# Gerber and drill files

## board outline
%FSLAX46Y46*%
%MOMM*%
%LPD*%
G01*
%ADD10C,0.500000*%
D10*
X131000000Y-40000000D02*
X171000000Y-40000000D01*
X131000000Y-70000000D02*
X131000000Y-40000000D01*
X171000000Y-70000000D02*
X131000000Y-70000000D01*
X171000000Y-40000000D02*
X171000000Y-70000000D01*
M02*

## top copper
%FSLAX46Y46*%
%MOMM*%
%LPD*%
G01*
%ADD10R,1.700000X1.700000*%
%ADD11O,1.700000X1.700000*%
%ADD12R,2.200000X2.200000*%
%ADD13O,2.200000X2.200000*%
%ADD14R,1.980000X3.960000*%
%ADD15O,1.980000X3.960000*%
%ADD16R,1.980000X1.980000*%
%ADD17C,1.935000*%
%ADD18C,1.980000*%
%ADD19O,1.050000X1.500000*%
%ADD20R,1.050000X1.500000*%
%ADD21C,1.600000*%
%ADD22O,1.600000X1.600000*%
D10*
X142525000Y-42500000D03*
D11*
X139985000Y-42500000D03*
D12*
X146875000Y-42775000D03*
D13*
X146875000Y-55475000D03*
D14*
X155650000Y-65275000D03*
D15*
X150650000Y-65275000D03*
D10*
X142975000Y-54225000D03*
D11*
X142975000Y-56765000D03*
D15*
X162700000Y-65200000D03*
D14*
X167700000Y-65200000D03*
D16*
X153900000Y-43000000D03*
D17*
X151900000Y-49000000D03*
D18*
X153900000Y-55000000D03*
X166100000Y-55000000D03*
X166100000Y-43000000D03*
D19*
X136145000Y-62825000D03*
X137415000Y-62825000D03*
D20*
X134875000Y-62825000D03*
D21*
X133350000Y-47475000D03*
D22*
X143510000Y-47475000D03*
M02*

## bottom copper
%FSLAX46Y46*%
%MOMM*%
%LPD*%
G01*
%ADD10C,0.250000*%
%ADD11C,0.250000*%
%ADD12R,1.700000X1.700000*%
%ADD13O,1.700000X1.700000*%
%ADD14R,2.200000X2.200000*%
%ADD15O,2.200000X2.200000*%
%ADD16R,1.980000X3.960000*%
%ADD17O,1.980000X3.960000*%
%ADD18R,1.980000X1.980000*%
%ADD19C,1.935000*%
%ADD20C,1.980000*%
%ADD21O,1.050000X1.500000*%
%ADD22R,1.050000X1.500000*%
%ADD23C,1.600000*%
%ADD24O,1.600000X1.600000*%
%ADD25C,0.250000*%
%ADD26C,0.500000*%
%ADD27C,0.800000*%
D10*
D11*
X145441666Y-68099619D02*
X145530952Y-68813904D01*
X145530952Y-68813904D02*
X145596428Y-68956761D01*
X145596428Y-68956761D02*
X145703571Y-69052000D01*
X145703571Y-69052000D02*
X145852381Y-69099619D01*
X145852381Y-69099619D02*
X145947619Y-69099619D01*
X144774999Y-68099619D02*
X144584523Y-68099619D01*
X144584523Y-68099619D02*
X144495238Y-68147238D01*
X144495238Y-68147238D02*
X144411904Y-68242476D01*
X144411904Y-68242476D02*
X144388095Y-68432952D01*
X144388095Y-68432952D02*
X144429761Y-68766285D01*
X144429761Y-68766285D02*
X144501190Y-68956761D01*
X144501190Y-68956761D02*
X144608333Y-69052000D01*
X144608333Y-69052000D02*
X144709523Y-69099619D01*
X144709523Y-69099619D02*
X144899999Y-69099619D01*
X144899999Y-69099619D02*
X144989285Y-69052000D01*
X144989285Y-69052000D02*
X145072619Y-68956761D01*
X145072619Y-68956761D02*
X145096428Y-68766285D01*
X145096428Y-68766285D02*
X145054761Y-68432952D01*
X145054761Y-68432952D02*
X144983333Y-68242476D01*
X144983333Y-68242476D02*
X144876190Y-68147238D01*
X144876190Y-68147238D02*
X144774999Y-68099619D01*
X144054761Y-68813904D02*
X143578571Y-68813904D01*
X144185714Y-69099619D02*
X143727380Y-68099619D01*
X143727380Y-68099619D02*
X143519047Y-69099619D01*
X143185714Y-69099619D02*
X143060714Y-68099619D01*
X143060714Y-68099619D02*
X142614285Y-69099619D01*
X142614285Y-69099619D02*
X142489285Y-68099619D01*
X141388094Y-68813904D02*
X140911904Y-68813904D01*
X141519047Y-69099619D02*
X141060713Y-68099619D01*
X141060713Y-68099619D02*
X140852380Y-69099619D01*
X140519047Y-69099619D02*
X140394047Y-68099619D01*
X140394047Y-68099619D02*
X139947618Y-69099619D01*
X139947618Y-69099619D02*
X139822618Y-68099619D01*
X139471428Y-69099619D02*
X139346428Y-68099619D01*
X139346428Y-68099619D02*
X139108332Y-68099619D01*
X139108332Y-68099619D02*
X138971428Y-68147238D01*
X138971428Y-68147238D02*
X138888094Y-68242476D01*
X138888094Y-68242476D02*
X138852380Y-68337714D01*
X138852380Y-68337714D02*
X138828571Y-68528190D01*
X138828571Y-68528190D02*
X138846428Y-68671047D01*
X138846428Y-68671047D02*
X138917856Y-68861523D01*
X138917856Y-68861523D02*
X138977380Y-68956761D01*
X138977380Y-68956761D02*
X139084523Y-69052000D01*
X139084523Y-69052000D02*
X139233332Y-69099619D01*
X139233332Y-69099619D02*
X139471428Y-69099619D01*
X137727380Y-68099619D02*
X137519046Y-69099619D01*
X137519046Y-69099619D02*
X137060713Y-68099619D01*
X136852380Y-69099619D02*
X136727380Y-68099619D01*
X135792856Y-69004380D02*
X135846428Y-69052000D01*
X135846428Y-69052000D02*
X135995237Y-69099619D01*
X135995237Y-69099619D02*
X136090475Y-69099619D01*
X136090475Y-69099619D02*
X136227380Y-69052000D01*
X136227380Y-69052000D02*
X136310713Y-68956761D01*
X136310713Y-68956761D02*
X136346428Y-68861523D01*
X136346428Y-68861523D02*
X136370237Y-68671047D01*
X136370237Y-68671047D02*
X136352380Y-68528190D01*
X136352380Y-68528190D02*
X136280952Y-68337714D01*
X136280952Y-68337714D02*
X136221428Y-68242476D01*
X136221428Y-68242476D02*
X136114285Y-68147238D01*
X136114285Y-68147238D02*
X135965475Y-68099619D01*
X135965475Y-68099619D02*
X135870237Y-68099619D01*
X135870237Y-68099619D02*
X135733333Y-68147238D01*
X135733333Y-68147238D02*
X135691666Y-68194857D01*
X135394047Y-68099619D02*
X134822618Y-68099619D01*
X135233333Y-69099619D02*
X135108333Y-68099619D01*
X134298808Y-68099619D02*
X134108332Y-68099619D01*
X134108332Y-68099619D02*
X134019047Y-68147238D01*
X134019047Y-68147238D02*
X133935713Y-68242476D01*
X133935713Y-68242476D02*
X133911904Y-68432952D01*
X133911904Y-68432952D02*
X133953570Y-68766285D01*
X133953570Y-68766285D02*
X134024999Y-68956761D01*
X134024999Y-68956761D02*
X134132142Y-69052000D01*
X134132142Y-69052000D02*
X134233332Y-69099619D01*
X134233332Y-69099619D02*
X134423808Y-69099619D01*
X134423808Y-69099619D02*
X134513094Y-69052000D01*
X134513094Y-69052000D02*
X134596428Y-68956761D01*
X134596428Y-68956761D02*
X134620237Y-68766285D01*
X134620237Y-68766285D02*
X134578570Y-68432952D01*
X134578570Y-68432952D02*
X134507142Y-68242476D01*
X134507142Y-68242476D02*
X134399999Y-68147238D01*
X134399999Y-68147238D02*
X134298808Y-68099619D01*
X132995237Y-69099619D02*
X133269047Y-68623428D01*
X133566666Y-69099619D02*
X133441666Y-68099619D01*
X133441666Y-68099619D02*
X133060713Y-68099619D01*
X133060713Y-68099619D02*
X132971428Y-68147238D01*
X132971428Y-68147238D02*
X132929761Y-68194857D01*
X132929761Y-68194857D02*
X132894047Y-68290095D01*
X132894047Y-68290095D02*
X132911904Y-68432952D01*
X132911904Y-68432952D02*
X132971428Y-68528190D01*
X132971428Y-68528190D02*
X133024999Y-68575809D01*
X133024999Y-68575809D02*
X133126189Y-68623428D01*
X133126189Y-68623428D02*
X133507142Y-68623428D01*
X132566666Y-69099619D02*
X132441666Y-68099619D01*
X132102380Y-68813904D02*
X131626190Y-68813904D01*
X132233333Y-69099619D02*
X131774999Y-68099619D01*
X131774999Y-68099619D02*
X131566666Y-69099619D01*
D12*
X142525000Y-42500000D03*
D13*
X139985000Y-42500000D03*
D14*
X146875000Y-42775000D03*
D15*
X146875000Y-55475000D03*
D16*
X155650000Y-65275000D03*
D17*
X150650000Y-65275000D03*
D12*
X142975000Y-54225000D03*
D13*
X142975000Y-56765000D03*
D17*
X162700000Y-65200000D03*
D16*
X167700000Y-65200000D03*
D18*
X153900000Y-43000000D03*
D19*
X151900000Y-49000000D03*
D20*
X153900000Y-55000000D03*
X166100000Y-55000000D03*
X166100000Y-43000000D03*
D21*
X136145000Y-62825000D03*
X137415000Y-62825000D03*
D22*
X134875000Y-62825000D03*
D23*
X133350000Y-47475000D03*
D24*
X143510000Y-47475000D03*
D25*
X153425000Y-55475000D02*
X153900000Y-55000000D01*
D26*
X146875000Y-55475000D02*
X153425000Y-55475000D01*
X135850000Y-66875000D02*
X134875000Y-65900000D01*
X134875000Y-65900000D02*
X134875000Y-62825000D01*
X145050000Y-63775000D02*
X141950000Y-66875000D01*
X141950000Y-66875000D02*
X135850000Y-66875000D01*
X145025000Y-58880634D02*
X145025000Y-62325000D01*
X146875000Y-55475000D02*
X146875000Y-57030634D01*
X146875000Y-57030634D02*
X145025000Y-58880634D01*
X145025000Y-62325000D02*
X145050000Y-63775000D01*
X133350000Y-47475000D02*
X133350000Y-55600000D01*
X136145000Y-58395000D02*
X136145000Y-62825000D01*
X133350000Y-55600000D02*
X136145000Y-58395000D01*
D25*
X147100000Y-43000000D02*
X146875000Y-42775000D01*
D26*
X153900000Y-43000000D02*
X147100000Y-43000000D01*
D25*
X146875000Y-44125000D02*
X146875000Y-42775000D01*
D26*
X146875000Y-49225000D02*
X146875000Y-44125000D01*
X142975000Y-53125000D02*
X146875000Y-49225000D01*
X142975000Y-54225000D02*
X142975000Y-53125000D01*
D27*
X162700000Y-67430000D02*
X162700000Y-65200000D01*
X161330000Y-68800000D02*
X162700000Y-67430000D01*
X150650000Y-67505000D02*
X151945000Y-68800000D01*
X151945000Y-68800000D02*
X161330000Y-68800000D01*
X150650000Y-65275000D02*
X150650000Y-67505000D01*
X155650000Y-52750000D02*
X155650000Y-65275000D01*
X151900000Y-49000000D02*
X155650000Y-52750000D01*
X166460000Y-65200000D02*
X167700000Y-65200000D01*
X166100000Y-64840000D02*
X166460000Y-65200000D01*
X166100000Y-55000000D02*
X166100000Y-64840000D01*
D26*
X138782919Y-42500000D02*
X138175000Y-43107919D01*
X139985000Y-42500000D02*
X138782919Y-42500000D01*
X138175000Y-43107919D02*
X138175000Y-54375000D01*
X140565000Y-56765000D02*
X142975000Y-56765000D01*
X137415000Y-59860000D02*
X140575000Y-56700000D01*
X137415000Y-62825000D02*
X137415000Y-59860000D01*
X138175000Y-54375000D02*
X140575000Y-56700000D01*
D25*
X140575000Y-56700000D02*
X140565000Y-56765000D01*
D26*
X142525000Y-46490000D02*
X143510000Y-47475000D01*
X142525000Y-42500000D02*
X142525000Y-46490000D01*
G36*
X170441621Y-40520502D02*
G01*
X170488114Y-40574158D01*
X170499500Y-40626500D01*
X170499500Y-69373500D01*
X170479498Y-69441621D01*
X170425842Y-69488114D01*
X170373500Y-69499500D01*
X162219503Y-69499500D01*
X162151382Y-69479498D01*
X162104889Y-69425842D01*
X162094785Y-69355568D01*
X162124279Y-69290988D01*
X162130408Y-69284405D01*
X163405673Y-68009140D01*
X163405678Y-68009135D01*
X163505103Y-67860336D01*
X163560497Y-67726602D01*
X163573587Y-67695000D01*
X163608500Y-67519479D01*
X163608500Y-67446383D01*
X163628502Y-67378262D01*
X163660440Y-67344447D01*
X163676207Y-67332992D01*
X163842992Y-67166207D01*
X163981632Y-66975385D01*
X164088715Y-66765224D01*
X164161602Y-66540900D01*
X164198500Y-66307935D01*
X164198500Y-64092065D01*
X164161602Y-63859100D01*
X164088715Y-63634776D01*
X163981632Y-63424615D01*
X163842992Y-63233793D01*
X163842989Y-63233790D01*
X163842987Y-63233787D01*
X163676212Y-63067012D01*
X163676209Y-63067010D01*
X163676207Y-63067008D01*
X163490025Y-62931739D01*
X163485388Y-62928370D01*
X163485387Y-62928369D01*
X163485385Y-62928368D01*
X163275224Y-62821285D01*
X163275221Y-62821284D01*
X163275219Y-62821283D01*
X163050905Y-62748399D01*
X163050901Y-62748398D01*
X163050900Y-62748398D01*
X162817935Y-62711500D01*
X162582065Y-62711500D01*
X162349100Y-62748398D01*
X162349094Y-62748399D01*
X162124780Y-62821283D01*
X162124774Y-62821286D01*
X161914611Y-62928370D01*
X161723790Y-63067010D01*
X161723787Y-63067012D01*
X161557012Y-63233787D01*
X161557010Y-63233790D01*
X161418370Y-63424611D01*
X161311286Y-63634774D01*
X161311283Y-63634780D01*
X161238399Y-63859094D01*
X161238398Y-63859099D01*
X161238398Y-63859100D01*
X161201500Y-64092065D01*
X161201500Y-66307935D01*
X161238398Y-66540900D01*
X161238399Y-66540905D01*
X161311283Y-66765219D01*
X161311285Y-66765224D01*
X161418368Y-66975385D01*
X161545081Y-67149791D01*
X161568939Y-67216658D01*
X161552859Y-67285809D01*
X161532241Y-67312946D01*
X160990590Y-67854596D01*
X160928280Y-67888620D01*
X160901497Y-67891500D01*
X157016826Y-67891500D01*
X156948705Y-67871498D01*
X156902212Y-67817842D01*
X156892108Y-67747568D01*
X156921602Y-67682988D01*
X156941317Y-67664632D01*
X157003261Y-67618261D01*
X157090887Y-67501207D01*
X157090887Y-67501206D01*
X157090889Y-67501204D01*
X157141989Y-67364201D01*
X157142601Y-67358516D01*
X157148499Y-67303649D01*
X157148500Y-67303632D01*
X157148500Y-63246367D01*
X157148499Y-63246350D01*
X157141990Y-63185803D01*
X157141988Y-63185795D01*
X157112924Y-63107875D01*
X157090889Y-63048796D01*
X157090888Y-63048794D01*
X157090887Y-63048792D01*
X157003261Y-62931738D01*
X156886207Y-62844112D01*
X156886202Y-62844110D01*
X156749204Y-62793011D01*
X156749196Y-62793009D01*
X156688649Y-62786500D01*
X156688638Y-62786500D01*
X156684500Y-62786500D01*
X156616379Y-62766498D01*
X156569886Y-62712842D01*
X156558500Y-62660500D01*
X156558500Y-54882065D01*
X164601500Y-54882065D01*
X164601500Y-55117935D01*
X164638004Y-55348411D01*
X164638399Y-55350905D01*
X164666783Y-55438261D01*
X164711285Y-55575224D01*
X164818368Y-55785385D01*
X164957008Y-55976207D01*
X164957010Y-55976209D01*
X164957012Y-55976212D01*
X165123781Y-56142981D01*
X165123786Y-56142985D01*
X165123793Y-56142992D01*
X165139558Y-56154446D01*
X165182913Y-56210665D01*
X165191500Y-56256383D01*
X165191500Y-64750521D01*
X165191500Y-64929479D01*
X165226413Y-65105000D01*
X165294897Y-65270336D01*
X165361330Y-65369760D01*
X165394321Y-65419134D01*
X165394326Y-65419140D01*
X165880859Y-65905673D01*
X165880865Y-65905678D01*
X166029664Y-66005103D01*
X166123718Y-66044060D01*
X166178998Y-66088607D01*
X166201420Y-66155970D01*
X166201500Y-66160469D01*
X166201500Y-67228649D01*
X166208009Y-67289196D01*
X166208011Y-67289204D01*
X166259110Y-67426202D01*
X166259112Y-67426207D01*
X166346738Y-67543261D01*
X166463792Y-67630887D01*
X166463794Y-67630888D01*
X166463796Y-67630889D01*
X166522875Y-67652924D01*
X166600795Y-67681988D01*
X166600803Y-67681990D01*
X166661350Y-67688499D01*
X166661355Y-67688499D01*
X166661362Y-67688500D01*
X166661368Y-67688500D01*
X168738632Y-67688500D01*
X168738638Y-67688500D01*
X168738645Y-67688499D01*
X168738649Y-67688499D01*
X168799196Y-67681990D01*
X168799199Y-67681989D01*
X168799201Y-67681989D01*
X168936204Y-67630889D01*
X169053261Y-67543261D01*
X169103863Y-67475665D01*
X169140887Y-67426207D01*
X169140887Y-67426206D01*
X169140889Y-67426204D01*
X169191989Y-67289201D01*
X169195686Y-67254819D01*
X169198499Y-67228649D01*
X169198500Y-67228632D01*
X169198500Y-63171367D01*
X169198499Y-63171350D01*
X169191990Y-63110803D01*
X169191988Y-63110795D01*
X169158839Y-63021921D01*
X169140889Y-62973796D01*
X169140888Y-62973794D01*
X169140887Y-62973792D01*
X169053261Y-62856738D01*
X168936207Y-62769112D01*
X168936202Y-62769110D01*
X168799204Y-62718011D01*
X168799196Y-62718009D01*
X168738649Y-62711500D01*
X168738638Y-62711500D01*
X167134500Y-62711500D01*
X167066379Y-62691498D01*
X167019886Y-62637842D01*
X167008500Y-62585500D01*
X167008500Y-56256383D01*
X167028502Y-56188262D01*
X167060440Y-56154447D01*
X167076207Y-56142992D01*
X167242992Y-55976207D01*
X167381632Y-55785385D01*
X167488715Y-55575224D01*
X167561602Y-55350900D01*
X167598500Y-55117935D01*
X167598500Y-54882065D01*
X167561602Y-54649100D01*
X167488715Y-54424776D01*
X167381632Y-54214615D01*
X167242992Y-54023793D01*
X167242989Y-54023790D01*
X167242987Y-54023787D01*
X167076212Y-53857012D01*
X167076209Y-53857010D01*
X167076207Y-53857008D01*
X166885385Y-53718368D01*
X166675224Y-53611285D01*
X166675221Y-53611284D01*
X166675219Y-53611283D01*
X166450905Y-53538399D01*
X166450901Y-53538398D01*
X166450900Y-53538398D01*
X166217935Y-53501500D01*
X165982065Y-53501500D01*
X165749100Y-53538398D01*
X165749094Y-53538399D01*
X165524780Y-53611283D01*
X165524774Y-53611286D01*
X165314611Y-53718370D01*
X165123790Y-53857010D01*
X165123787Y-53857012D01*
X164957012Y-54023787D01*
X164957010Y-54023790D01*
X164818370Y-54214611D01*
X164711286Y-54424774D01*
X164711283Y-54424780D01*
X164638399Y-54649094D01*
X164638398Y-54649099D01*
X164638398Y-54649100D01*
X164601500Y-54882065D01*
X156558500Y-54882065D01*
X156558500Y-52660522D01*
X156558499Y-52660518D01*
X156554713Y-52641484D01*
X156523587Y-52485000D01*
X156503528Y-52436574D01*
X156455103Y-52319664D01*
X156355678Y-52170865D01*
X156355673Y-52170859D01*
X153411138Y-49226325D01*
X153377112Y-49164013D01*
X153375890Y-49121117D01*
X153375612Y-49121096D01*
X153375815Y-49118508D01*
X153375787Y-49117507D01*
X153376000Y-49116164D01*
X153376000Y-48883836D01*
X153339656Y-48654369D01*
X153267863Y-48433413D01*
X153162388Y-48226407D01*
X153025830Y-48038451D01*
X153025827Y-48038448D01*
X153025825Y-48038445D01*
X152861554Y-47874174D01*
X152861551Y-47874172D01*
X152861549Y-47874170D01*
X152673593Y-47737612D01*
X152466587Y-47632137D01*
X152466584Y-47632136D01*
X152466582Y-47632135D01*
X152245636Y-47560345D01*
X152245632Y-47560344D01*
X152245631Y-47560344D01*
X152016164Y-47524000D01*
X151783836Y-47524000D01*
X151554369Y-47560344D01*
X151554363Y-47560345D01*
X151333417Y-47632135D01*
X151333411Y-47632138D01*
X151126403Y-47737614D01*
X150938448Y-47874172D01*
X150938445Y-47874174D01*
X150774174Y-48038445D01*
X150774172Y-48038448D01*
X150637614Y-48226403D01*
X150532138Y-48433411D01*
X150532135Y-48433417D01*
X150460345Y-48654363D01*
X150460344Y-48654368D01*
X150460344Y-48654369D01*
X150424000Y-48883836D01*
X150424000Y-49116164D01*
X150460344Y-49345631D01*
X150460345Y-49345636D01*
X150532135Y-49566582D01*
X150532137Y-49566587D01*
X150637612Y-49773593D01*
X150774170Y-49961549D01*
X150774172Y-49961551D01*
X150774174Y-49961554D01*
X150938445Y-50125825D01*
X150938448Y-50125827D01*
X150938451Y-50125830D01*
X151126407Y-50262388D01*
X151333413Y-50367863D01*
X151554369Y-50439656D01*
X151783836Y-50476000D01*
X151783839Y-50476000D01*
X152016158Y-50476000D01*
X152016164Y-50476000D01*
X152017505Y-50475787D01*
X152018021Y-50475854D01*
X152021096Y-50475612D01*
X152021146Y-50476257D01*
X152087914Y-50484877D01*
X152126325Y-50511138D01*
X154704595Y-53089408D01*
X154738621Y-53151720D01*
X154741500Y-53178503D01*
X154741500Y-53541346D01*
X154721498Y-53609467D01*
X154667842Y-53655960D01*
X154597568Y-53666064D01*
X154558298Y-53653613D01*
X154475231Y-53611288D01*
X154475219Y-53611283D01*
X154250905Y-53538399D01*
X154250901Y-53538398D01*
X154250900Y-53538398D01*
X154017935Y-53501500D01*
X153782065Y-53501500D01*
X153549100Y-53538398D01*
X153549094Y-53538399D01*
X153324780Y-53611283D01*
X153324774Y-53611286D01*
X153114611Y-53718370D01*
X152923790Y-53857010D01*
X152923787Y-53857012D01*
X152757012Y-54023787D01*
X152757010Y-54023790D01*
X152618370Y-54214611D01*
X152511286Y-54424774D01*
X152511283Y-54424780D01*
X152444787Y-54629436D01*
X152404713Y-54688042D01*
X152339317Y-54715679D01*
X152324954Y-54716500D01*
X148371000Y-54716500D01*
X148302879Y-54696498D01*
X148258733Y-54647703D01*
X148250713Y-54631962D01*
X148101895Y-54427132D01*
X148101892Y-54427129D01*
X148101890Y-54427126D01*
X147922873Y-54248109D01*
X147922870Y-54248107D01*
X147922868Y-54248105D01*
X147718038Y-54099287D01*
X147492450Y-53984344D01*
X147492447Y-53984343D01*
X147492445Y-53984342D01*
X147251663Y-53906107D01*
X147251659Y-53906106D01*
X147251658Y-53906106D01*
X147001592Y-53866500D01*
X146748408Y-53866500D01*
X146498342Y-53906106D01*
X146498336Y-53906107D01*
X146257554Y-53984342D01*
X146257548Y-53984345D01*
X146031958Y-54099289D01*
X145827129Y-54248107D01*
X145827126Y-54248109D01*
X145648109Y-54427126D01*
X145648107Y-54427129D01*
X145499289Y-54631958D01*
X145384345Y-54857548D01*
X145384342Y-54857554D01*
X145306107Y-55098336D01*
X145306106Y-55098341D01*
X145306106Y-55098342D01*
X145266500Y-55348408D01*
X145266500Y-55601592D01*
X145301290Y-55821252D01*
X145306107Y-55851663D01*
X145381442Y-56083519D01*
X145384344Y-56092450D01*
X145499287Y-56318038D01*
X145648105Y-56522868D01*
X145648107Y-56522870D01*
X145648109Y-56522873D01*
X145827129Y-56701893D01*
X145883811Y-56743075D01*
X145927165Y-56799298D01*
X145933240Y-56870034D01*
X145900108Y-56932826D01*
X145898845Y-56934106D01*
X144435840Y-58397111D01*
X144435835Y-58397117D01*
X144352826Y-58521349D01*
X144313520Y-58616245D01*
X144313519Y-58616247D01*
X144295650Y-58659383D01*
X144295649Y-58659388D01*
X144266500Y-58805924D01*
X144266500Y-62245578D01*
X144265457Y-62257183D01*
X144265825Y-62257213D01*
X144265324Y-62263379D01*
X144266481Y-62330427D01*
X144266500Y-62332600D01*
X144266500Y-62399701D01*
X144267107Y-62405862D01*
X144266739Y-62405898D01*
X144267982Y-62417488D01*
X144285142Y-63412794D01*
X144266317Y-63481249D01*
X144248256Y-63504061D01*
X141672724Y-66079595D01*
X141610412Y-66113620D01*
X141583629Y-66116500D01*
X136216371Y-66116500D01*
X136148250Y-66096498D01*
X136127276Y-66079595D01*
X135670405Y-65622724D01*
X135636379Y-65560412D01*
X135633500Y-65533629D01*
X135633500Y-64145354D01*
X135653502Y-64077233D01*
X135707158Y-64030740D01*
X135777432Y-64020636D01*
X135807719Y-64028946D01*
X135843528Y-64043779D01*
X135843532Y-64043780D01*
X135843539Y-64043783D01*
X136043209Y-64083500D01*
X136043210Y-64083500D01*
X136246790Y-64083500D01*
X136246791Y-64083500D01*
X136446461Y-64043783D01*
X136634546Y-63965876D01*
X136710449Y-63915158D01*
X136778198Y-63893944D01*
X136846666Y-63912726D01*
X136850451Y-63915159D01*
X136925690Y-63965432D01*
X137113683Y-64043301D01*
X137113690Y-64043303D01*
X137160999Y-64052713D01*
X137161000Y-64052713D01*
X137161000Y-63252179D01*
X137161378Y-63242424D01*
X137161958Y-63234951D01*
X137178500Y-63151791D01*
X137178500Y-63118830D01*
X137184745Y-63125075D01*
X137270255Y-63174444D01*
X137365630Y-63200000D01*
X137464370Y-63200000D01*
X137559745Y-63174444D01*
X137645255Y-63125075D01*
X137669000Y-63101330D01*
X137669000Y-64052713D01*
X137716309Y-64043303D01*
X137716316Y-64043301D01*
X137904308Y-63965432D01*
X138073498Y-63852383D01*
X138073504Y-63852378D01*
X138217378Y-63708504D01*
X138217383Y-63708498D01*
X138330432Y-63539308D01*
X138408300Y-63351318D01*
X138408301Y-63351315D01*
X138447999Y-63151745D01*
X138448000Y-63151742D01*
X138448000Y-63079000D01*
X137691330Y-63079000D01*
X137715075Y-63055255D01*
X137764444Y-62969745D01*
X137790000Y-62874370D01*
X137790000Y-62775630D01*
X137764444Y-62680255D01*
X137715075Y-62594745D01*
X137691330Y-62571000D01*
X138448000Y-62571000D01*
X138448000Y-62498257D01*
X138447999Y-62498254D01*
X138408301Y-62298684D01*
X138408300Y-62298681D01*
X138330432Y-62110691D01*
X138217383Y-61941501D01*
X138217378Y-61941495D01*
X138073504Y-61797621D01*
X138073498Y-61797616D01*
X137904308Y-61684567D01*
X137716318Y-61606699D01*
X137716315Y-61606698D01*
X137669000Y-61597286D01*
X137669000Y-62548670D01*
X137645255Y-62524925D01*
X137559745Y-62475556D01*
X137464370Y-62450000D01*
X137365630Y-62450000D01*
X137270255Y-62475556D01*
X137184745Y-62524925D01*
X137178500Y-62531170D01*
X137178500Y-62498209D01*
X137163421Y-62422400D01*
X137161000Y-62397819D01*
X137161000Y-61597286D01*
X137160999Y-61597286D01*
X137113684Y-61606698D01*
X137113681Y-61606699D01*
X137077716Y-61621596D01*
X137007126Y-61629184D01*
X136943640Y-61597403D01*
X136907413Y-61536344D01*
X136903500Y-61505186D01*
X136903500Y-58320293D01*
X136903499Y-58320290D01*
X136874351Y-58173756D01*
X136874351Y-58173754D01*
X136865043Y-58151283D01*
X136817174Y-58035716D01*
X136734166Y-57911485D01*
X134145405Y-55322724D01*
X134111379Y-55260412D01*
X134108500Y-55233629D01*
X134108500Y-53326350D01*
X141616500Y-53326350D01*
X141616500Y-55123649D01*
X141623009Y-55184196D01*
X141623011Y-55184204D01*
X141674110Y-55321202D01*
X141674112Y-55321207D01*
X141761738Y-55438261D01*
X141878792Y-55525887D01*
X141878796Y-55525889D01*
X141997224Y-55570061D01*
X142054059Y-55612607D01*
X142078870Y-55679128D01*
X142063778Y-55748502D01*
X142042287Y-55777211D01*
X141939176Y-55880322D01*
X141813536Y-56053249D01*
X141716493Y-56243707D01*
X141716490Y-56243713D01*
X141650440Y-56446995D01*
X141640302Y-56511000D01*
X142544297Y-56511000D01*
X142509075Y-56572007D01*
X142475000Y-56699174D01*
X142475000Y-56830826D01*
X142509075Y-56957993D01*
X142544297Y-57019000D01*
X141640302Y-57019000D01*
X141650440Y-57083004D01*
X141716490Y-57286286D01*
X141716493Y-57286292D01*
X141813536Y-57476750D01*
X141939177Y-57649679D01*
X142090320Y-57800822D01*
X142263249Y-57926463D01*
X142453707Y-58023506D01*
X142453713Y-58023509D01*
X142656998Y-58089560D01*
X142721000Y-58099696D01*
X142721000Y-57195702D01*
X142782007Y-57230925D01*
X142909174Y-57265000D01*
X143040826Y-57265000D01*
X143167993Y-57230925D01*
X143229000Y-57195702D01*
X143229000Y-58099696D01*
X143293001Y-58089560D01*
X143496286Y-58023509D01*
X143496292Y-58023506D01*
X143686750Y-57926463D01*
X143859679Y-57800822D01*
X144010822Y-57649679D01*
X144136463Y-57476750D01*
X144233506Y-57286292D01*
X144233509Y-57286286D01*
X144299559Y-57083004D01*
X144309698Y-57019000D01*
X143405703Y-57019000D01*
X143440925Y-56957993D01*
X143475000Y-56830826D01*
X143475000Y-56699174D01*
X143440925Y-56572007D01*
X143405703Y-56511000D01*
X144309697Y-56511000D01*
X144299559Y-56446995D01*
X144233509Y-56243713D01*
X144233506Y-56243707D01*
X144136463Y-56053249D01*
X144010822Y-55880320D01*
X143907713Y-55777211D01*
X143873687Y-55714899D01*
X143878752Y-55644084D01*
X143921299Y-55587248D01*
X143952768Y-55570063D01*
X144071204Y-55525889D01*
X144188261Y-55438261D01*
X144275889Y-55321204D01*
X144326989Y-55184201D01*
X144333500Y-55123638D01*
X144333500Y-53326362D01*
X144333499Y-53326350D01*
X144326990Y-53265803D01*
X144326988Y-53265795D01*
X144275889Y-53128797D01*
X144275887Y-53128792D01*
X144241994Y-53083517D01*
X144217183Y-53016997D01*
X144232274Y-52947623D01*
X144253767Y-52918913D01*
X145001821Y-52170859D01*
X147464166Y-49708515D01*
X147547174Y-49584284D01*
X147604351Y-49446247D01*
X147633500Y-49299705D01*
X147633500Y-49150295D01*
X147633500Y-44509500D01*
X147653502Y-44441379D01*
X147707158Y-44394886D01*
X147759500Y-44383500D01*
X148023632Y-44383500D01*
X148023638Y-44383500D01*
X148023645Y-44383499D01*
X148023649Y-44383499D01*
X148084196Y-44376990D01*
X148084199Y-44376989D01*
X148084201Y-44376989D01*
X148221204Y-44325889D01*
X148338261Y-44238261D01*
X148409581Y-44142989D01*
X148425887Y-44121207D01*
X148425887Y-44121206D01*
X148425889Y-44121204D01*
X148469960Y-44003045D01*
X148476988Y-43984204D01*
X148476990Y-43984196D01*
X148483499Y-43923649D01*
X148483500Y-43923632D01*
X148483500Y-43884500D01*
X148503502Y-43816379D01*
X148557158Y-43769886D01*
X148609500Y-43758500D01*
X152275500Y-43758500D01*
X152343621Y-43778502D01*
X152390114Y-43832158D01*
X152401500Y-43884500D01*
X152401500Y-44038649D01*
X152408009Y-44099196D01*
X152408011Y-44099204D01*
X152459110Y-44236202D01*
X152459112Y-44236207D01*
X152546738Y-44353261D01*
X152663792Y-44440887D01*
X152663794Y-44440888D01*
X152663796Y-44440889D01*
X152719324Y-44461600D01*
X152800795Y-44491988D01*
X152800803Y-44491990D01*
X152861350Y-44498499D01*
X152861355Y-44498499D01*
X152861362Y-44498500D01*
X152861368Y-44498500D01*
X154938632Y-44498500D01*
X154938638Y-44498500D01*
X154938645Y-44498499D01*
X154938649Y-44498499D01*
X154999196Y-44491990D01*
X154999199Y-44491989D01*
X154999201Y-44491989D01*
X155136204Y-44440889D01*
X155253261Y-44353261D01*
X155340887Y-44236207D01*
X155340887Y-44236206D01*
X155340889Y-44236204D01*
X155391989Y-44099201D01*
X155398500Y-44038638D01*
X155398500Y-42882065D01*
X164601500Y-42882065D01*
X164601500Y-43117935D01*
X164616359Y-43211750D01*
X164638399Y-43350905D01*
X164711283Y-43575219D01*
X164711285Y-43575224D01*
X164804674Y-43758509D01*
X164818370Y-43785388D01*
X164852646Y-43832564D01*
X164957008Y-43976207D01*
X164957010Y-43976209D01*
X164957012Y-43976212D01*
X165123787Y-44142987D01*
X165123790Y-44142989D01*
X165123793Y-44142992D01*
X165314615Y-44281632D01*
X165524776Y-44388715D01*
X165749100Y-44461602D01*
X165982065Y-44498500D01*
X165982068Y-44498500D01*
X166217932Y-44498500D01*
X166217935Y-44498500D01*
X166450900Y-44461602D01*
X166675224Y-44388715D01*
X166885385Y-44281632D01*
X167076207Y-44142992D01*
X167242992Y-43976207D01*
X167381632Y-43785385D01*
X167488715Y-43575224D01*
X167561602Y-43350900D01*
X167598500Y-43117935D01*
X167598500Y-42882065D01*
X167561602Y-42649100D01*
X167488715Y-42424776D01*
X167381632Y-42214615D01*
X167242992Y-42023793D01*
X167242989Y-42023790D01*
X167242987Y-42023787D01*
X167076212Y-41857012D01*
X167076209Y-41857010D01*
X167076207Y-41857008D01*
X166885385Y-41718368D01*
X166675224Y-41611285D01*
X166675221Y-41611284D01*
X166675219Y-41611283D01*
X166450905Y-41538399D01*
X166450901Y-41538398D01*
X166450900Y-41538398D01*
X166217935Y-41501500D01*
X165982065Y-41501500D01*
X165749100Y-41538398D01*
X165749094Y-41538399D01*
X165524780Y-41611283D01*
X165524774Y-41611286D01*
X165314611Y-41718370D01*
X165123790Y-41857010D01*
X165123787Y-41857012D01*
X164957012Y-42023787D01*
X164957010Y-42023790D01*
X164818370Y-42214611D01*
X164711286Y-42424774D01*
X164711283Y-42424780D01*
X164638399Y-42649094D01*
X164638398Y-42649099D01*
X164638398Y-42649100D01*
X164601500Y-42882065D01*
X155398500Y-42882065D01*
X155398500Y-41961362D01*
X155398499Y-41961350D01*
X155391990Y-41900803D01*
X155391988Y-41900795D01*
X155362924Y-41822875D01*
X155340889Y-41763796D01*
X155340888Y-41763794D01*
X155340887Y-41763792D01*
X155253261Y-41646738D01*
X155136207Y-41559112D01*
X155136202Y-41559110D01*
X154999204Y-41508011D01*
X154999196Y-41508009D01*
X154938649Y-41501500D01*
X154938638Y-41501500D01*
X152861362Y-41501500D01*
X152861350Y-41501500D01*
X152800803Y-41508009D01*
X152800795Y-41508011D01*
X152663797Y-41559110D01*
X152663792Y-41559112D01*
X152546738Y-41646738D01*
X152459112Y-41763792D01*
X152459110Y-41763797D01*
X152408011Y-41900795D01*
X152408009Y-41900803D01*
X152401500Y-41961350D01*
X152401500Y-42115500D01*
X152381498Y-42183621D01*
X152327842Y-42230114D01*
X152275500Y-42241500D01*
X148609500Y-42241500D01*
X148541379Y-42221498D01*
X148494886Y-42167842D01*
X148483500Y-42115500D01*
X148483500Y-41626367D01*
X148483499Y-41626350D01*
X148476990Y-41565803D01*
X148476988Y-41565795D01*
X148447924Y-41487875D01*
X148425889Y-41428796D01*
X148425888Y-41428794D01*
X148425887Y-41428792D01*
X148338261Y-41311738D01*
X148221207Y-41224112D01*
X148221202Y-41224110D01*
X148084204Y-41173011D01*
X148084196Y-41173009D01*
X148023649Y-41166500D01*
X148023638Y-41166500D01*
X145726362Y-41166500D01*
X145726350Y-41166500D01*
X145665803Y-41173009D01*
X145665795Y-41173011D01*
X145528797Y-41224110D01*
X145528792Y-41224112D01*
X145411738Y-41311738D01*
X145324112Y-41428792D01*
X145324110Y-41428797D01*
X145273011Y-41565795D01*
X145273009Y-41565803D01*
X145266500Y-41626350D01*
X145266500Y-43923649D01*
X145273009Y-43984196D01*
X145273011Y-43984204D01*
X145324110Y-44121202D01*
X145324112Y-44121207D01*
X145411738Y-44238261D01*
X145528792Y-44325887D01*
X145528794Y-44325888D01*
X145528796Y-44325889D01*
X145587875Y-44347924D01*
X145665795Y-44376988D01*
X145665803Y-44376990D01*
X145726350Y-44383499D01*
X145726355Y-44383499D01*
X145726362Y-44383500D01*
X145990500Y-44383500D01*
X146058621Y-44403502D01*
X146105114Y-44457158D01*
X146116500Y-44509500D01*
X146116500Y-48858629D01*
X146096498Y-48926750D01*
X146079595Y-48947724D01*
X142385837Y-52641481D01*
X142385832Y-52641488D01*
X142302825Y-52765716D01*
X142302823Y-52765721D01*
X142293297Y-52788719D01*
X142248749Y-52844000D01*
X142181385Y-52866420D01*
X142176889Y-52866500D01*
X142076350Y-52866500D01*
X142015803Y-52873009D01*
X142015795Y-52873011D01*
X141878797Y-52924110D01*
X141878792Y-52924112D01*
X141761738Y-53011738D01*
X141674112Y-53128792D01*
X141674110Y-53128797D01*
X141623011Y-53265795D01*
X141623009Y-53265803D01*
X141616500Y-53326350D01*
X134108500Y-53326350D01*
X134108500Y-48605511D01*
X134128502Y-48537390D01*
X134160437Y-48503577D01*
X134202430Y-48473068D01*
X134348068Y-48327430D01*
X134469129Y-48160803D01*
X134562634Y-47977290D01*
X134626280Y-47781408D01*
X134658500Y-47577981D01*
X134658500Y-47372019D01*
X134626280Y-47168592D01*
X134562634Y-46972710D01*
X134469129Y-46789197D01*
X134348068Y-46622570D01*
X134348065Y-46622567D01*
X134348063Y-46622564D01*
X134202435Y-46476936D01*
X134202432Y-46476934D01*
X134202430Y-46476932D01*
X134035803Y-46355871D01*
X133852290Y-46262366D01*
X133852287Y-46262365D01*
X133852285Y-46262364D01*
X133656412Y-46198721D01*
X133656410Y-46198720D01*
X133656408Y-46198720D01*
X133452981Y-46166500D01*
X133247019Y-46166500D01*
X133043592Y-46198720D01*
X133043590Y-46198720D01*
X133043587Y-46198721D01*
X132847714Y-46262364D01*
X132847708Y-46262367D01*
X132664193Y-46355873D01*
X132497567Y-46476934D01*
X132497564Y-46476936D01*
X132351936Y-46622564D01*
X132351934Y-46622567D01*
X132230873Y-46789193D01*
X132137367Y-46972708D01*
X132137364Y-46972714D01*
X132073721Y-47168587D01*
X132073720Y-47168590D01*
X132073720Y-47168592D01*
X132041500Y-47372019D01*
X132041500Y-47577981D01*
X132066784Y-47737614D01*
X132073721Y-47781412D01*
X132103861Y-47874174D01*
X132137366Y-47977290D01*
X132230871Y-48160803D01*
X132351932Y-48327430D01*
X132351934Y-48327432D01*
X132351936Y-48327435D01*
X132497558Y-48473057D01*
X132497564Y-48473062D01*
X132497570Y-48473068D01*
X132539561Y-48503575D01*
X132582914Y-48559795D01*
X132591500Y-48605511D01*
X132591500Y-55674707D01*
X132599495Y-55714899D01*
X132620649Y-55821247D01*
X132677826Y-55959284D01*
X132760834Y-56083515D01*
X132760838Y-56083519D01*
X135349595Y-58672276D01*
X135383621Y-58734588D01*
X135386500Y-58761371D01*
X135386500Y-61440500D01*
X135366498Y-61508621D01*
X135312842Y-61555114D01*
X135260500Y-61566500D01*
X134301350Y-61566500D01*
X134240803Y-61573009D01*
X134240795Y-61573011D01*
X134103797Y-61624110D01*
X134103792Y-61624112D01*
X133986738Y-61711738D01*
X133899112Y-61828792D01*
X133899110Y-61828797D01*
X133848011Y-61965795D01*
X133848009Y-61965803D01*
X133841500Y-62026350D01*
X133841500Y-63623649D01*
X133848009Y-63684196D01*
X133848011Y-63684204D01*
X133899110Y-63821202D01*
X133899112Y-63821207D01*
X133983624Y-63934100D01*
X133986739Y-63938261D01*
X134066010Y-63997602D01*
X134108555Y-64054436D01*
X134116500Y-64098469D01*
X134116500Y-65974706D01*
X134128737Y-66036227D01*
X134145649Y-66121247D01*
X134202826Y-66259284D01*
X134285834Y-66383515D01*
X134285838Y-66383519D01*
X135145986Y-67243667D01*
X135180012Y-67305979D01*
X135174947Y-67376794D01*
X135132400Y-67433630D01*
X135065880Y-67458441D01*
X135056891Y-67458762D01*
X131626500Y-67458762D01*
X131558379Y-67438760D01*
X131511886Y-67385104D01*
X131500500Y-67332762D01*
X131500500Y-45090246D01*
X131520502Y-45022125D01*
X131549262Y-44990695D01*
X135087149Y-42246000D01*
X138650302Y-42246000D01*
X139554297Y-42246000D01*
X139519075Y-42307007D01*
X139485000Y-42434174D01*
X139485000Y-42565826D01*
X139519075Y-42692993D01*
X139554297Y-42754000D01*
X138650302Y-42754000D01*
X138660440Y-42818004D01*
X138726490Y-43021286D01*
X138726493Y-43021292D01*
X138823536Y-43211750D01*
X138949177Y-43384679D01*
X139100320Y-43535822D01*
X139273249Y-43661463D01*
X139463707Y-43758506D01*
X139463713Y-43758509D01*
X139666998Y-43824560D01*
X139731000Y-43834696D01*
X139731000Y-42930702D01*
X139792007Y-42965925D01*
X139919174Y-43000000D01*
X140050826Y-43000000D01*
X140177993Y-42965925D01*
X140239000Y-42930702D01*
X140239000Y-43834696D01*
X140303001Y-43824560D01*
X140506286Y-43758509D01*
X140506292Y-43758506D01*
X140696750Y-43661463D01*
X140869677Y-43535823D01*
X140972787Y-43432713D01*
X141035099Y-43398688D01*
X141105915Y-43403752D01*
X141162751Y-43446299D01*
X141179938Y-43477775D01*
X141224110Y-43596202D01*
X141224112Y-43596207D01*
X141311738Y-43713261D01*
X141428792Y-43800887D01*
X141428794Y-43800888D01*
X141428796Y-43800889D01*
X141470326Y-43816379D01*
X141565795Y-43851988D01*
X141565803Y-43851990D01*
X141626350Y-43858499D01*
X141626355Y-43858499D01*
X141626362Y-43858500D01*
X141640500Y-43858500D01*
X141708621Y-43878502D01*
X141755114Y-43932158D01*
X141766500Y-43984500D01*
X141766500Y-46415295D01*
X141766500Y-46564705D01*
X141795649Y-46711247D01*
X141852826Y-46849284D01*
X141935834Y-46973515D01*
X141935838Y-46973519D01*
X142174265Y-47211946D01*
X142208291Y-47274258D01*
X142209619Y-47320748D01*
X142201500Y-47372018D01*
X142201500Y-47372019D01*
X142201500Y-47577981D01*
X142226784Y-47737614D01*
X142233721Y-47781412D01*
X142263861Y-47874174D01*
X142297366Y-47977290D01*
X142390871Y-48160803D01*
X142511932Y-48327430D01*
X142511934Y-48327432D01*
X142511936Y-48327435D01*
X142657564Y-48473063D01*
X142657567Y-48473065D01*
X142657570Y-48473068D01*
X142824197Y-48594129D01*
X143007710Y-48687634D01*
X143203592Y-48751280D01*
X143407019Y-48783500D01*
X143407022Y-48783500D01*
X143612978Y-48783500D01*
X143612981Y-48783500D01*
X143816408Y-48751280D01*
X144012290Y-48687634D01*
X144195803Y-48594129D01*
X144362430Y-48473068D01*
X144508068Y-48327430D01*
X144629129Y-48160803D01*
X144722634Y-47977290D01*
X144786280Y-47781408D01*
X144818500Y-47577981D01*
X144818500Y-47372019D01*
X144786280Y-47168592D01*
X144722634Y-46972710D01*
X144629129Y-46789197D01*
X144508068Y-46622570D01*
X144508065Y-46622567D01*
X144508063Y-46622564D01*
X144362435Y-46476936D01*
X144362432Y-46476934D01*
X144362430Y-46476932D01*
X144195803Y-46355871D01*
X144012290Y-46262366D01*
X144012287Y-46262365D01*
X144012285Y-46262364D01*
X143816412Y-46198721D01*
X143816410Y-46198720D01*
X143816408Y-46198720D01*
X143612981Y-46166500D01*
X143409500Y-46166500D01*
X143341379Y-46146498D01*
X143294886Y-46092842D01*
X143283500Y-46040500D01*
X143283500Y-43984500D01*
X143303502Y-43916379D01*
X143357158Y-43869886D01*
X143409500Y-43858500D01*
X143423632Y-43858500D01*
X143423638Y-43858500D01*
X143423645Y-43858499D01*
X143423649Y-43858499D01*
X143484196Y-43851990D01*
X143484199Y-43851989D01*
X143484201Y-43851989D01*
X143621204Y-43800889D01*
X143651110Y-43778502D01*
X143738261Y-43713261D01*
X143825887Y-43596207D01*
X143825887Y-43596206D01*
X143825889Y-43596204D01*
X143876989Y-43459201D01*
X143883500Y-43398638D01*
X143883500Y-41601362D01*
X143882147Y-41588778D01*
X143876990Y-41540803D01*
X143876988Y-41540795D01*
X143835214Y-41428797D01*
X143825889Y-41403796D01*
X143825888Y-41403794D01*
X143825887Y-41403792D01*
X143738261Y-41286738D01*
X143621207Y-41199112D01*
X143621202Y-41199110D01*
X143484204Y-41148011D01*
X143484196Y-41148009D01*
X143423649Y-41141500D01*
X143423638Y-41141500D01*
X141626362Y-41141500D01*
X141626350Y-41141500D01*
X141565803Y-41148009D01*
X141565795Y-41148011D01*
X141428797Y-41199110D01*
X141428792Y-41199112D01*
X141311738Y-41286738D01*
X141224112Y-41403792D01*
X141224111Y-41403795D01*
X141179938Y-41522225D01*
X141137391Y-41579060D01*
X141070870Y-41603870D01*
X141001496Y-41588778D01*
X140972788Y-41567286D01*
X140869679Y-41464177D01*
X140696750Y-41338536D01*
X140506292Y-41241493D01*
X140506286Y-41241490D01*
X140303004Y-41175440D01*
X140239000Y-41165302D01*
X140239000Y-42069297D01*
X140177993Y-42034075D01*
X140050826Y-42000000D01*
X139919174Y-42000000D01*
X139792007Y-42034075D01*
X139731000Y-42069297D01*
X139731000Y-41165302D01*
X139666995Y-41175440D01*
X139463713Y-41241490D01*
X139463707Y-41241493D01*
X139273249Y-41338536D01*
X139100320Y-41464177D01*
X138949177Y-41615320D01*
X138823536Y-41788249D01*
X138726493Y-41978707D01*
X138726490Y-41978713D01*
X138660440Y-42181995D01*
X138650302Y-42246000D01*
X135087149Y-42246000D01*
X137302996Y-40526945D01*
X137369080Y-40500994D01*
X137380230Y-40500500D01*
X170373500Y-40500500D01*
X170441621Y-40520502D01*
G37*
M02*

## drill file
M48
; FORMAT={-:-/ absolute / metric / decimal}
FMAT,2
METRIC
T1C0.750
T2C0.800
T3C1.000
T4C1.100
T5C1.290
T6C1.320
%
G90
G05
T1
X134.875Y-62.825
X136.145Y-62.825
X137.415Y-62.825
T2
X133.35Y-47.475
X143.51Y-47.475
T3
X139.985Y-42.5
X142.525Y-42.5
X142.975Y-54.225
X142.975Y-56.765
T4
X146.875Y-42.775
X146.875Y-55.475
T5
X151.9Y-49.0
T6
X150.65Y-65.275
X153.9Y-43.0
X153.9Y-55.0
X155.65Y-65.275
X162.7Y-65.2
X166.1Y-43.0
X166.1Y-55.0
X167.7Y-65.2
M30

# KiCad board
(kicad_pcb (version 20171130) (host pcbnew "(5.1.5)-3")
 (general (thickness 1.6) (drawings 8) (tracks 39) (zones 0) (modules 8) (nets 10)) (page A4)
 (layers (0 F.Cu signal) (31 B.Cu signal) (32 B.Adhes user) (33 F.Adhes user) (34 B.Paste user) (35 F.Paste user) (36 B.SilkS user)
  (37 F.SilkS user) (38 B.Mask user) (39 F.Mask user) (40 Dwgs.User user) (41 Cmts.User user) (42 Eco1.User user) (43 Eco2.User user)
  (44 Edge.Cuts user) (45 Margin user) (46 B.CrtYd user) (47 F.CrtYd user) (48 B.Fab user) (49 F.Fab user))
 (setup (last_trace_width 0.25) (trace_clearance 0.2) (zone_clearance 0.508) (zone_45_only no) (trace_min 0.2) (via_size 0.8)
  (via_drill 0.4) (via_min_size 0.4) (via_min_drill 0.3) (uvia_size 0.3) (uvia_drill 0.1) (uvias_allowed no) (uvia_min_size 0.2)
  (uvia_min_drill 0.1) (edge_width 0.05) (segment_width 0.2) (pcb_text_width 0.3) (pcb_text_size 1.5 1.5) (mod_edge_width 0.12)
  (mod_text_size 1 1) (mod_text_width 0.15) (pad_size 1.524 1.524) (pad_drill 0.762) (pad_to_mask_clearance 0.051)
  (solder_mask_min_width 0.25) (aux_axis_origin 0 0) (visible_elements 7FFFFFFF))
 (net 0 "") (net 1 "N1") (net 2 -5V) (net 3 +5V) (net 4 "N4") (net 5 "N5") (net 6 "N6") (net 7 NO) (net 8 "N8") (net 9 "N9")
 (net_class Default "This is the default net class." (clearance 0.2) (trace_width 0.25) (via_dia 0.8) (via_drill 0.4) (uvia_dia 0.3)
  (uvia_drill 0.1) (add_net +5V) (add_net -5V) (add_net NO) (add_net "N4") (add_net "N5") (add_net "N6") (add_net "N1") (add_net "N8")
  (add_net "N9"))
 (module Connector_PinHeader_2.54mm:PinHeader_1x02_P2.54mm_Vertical (layer F.Cu) (at 142.525 42.5 270)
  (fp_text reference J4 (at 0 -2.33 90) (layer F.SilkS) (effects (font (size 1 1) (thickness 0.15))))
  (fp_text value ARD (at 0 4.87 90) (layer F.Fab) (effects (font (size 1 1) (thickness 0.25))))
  (pad 1 thru_hole rect (at 0 0 270) (size 1.7 1.7) (drill 1) (layers *.Cu *.Mask) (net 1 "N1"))
  (pad 2 thru_hole oval (at 0 2.54 270) (size 1.7 1.7) (drill 1) (layers *.Cu *.Mask) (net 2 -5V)))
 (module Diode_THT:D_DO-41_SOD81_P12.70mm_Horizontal (layer F.Cu) (at 146.875 42.775 270)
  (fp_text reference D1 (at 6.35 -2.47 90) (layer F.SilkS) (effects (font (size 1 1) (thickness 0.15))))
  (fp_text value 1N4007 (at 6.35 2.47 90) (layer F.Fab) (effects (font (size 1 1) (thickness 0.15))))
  (pad 1 thru_hole rect (at 0 0 270) (size 2.2 2.2) (drill 1.1) (layers *.Cu *.Mask) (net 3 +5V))
  (pad 2 thru_hole oval (at 12.7 0 270) (size 2.2 2.2) (drill 1.1) (layers *.Cu *.Mask) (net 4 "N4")))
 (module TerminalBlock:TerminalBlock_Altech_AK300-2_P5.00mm (layer F.Cu) (at 155.65 65.275 180)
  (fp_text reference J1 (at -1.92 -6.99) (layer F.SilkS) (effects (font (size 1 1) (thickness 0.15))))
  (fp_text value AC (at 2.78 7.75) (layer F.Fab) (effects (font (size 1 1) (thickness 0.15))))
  (pad 1 thru_hole rect (at 0 0 180) (size 1.98 3.96) (drill 1.32) (layers *.Cu *.Mask) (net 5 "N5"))
  (pad 2 thru_hole oval (at 5 0 180) (size 1.98 3.96) (drill 1.32) (layers *.Cu *.Mask) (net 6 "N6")))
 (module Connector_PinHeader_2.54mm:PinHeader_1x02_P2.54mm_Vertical (layer F.Cu) (at 142.975 54.225)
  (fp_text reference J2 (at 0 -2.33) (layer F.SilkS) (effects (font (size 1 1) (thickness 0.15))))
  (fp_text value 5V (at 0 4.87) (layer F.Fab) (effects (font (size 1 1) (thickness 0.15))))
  (pad 1 thru_hole rect (at 0 0) (size 1.7 1.7) (drill 1) (layers *.Cu *.Mask) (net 3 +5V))
  (pad 2 thru_hole oval (at 0 2.54) (size 1.7 1.7) (drill 1) (layers *.Cu *.Mask) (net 2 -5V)))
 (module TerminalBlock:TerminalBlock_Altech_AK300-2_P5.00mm (layer F.Cu) (at 167.7 65.2 180)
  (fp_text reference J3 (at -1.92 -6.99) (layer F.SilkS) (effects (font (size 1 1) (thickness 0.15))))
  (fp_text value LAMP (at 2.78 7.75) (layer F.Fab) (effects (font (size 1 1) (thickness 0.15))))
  (pad 2 thru_hole oval (at 5 0 180) (size 1.98 3.96) (drill 1.32) (layers *.Cu *.Mask) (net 6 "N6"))
  (pad 1 thru_hole rect (at 0 0 180) (size 1.98 3.96) (drill 1.32) (layers *.Cu *.Mask) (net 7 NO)))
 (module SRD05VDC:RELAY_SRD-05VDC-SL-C (layer F.Cu) (at 160 49)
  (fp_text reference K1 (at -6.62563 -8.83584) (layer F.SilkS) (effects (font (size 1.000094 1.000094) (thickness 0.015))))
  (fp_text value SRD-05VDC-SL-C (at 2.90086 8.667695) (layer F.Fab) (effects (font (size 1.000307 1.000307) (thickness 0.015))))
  (pad A1 thru_hole rect (at -6.1 -6) (size 1.98 1.98) (drill 1.32) (layers *.Cu *.Mask) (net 3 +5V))
  (pad COM thru_hole circle (at -8.1 0) (size 1.935 1.935) (drill 1.29) (layers *.Cu *.Mask) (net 5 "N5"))
  (pad A2 thru_hole circle (at -6.1 6) (size 1.98 1.98) (drill 1.32) (layers *.Cu *.Mask) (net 4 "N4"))
  (pad NO thru_hole circle (at 6.1 6) (size 1.98 1.98) (drill 1.32) (layers *.Cu *.Mask) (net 7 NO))
  (pad NC thru_hole circle (at 6.1 -6) (size 1.98 1.98) (drill 1.32) (layers *.Cu *.Mask) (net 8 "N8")))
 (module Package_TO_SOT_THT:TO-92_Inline (layer F.Cu) (at 134.875 62.825)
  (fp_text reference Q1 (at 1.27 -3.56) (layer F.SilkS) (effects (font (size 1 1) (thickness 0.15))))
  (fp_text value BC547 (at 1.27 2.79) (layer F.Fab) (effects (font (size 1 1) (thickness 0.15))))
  (pad 2 thru_hole oval (at 1.27 0) (size 1.05 1.5) (drill 0.75) (layers *.Cu *.Mask) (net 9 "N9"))
  (pad 3 thru_hole oval (at 2.54 0) (size 1.05 1.5) (drill 0.75) (layers *.Cu *.Mask) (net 2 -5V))
  (pad 1 thru_hole rect (at 0 0) (size 1.05 1.5) (drill 0.75) (layers *.Cu *.Mask) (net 4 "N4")))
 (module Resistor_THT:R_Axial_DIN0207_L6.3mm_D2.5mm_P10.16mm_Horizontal (layer F.Cu) (at 133.35 47.475)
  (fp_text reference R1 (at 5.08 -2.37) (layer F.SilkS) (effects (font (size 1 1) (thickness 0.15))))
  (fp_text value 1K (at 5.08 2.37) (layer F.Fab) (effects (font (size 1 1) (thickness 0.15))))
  (pad 1 thru_hole circle (at 0 0) (size 1.6 1.6) (drill 0.8) (layers *.Cu *.Mask) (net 9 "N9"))
  (pad 2 thru_hole oval (at 10.16 0) (size 1.6 1.6) (drill 0.8) (layers *.Cu *.Mask) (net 1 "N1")))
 (gr_line (start 131 40) (end 171 40) (layer Edge.Cuts) (width 0.5))
 (gr_line (start 131 70) (end 131 40) (layer Edge.Cuts) (width 0.5))
 (gr_line (start 171 70) (end 131 70) (layer Edge.Cuts) (width 0.5))
 (gr_line (start 171 40) (end 171 70) (layer Edge.Cuts) (width 0.5))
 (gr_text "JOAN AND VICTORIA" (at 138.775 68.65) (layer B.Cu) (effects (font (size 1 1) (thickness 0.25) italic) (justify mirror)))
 (segment (start 153.425 55.475) (end 153.9 55) (width 0.25) (layer B.Cu) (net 4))
 (segment (start 146.875 55.475) (end 153.425 55.475) (width 0.5) (layer B.Cu) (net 4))
 (segment (start 135.85 66.875) (end 134.875 65.9) (width 0.5) (layer B.Cu) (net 4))
 (segment (start 134.875 65.9) (end 134.875 62.825) (width 0.5) (layer B.Cu) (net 4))
 (segment (start 145.05 63.775) (end 141.95 66.875) (width 0.5) (layer B.Cu) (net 4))
 (segment (start 141.95 66.875) (end 135.85 66.875) (width 0.5) (layer B.Cu) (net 4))
 (segment (start 145.025 58.880634) (end 145.025 62.325) (width 0.5) (layer B.Cu) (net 4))
 (segment (start 146.875 55.475) (end 146.875 57.030634) (width 0.5) (layer B.Cu) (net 4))
 (segment (start 146.875 57.030634) (end 145.025 58.880634) (width 0.5) (layer B.Cu) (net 4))
 (segment (start 145.025 62.325) (end 145.05 63.775) (width 0.5) (layer B.Cu) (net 4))
 (segment (start 133.35 47.475) (end 133.35 55.6) (width 0.5) (layer B.Cu) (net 9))
 (segment (start 136.145 58.395) (end 136.145 62.825) (width 0.5) (layer B.Cu) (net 9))
 (segment (start 133.35 55.6) (end 136.145 58.395) (width 0.5) (layer B.Cu) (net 9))
 (segment (start 147.1 43) (end 146.875 42.775) (width 0.25) (layer B.Cu) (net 3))
 (segment (start 153.9 43) (end 147.1 43) (width 0.5) (layer B.Cu) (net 3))
 (segment (start 146.875 44.125) (end 146.875 42.775) (width 0.25) (layer B.Cu) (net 3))
 (segment (start 146.875 49.225) (end 146.875 44.125) (width 0.5) (layer B.Cu) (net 3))
 (segment (start 142.975 53.125) (end 146.875 49.225) (width 0.5) (layer B.Cu) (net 3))
 (segment (start 142.975 54.225) (end 142.975 53.125) (width 0.5) (layer B.Cu) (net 3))
 (segment (start 162.7 67.43) (end 162.7 65.2) (width 0.8) (layer B.Cu) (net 6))
 (segment (start 161.33 68.8) (end 162.7 67.43) (width 0.8) (layer B.Cu) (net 6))
 (segment (start 150.65 67.505) (end 151.945 68.8) (width 0.8) (layer B.Cu) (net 6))
 (segment (start 151.945 68.8) (end 161.33 68.8) (width 0.8) (layer B.Cu) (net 6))
 (segment (start 150.65 65.275) (end 150.65 67.505) (width 0.8) (layer B.Cu) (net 6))
 (segment (start 155.65 52.75) (end 155.65 65.275) (width 0.8) (layer B.Cu) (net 5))
 (segment (start 151.9 49) (end 155.65 52.75) (width 0.8) (layer B.Cu) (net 5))
 (segment (start 166.46 65.2) (end 167.7 65.2) (width 0.8) (layer B.Cu) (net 7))
 (segment (start 166.1 64.84) (end 166.46 65.2) (width 0.8) (layer B.Cu) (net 7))
 (segment (start 166.1 55) (end 166.1 64.84) (width 0.8) (layer B.Cu) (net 7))
 (segment (start 138.782919 42.5) (end 138.175 43.107919) (width 0.5) (layer B.Cu) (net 2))
 (segment (start 139.985 42.5) (end 138.782919 42.5) (width 0.5) (layer B.Cu) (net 2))
 (segment (start 138.175 43.107919) (end 138.175 54.375) (width 0.5) (layer B.Cu) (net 2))
 (segment (start 140.565 56.765) (end 142.975 56.765) (width 0.5) (layer B.Cu) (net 2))
 (segment (start 137.415 59.86) (end 140.575 56.7) (width 0.5) (layer B.Cu) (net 2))
 (segment (start 137.415 62.825) (end 137.415 59.86) (width 0.5) (layer B.Cu) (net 2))
 (segment (start 138.175 54.375) (end 140.575 56.7) (width 0.5) (layer B.Cu) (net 2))
 (segment (start 140.575 56.7) (end 140.565 56.765) (width 0.25) (layer B.Cu) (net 2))
 (segment (start 142.525 46.49) (end 143.51 47.475) (width 0.5) (layer B.Cu) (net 1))
 (segment (start 142.525 42.5) (end 142.525 46.49) (width 0.5) (layer B.Cu) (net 1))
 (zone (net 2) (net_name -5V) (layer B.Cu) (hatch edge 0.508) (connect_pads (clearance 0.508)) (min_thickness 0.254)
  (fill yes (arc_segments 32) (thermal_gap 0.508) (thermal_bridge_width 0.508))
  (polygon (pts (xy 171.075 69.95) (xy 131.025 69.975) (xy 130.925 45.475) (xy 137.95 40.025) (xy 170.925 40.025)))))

